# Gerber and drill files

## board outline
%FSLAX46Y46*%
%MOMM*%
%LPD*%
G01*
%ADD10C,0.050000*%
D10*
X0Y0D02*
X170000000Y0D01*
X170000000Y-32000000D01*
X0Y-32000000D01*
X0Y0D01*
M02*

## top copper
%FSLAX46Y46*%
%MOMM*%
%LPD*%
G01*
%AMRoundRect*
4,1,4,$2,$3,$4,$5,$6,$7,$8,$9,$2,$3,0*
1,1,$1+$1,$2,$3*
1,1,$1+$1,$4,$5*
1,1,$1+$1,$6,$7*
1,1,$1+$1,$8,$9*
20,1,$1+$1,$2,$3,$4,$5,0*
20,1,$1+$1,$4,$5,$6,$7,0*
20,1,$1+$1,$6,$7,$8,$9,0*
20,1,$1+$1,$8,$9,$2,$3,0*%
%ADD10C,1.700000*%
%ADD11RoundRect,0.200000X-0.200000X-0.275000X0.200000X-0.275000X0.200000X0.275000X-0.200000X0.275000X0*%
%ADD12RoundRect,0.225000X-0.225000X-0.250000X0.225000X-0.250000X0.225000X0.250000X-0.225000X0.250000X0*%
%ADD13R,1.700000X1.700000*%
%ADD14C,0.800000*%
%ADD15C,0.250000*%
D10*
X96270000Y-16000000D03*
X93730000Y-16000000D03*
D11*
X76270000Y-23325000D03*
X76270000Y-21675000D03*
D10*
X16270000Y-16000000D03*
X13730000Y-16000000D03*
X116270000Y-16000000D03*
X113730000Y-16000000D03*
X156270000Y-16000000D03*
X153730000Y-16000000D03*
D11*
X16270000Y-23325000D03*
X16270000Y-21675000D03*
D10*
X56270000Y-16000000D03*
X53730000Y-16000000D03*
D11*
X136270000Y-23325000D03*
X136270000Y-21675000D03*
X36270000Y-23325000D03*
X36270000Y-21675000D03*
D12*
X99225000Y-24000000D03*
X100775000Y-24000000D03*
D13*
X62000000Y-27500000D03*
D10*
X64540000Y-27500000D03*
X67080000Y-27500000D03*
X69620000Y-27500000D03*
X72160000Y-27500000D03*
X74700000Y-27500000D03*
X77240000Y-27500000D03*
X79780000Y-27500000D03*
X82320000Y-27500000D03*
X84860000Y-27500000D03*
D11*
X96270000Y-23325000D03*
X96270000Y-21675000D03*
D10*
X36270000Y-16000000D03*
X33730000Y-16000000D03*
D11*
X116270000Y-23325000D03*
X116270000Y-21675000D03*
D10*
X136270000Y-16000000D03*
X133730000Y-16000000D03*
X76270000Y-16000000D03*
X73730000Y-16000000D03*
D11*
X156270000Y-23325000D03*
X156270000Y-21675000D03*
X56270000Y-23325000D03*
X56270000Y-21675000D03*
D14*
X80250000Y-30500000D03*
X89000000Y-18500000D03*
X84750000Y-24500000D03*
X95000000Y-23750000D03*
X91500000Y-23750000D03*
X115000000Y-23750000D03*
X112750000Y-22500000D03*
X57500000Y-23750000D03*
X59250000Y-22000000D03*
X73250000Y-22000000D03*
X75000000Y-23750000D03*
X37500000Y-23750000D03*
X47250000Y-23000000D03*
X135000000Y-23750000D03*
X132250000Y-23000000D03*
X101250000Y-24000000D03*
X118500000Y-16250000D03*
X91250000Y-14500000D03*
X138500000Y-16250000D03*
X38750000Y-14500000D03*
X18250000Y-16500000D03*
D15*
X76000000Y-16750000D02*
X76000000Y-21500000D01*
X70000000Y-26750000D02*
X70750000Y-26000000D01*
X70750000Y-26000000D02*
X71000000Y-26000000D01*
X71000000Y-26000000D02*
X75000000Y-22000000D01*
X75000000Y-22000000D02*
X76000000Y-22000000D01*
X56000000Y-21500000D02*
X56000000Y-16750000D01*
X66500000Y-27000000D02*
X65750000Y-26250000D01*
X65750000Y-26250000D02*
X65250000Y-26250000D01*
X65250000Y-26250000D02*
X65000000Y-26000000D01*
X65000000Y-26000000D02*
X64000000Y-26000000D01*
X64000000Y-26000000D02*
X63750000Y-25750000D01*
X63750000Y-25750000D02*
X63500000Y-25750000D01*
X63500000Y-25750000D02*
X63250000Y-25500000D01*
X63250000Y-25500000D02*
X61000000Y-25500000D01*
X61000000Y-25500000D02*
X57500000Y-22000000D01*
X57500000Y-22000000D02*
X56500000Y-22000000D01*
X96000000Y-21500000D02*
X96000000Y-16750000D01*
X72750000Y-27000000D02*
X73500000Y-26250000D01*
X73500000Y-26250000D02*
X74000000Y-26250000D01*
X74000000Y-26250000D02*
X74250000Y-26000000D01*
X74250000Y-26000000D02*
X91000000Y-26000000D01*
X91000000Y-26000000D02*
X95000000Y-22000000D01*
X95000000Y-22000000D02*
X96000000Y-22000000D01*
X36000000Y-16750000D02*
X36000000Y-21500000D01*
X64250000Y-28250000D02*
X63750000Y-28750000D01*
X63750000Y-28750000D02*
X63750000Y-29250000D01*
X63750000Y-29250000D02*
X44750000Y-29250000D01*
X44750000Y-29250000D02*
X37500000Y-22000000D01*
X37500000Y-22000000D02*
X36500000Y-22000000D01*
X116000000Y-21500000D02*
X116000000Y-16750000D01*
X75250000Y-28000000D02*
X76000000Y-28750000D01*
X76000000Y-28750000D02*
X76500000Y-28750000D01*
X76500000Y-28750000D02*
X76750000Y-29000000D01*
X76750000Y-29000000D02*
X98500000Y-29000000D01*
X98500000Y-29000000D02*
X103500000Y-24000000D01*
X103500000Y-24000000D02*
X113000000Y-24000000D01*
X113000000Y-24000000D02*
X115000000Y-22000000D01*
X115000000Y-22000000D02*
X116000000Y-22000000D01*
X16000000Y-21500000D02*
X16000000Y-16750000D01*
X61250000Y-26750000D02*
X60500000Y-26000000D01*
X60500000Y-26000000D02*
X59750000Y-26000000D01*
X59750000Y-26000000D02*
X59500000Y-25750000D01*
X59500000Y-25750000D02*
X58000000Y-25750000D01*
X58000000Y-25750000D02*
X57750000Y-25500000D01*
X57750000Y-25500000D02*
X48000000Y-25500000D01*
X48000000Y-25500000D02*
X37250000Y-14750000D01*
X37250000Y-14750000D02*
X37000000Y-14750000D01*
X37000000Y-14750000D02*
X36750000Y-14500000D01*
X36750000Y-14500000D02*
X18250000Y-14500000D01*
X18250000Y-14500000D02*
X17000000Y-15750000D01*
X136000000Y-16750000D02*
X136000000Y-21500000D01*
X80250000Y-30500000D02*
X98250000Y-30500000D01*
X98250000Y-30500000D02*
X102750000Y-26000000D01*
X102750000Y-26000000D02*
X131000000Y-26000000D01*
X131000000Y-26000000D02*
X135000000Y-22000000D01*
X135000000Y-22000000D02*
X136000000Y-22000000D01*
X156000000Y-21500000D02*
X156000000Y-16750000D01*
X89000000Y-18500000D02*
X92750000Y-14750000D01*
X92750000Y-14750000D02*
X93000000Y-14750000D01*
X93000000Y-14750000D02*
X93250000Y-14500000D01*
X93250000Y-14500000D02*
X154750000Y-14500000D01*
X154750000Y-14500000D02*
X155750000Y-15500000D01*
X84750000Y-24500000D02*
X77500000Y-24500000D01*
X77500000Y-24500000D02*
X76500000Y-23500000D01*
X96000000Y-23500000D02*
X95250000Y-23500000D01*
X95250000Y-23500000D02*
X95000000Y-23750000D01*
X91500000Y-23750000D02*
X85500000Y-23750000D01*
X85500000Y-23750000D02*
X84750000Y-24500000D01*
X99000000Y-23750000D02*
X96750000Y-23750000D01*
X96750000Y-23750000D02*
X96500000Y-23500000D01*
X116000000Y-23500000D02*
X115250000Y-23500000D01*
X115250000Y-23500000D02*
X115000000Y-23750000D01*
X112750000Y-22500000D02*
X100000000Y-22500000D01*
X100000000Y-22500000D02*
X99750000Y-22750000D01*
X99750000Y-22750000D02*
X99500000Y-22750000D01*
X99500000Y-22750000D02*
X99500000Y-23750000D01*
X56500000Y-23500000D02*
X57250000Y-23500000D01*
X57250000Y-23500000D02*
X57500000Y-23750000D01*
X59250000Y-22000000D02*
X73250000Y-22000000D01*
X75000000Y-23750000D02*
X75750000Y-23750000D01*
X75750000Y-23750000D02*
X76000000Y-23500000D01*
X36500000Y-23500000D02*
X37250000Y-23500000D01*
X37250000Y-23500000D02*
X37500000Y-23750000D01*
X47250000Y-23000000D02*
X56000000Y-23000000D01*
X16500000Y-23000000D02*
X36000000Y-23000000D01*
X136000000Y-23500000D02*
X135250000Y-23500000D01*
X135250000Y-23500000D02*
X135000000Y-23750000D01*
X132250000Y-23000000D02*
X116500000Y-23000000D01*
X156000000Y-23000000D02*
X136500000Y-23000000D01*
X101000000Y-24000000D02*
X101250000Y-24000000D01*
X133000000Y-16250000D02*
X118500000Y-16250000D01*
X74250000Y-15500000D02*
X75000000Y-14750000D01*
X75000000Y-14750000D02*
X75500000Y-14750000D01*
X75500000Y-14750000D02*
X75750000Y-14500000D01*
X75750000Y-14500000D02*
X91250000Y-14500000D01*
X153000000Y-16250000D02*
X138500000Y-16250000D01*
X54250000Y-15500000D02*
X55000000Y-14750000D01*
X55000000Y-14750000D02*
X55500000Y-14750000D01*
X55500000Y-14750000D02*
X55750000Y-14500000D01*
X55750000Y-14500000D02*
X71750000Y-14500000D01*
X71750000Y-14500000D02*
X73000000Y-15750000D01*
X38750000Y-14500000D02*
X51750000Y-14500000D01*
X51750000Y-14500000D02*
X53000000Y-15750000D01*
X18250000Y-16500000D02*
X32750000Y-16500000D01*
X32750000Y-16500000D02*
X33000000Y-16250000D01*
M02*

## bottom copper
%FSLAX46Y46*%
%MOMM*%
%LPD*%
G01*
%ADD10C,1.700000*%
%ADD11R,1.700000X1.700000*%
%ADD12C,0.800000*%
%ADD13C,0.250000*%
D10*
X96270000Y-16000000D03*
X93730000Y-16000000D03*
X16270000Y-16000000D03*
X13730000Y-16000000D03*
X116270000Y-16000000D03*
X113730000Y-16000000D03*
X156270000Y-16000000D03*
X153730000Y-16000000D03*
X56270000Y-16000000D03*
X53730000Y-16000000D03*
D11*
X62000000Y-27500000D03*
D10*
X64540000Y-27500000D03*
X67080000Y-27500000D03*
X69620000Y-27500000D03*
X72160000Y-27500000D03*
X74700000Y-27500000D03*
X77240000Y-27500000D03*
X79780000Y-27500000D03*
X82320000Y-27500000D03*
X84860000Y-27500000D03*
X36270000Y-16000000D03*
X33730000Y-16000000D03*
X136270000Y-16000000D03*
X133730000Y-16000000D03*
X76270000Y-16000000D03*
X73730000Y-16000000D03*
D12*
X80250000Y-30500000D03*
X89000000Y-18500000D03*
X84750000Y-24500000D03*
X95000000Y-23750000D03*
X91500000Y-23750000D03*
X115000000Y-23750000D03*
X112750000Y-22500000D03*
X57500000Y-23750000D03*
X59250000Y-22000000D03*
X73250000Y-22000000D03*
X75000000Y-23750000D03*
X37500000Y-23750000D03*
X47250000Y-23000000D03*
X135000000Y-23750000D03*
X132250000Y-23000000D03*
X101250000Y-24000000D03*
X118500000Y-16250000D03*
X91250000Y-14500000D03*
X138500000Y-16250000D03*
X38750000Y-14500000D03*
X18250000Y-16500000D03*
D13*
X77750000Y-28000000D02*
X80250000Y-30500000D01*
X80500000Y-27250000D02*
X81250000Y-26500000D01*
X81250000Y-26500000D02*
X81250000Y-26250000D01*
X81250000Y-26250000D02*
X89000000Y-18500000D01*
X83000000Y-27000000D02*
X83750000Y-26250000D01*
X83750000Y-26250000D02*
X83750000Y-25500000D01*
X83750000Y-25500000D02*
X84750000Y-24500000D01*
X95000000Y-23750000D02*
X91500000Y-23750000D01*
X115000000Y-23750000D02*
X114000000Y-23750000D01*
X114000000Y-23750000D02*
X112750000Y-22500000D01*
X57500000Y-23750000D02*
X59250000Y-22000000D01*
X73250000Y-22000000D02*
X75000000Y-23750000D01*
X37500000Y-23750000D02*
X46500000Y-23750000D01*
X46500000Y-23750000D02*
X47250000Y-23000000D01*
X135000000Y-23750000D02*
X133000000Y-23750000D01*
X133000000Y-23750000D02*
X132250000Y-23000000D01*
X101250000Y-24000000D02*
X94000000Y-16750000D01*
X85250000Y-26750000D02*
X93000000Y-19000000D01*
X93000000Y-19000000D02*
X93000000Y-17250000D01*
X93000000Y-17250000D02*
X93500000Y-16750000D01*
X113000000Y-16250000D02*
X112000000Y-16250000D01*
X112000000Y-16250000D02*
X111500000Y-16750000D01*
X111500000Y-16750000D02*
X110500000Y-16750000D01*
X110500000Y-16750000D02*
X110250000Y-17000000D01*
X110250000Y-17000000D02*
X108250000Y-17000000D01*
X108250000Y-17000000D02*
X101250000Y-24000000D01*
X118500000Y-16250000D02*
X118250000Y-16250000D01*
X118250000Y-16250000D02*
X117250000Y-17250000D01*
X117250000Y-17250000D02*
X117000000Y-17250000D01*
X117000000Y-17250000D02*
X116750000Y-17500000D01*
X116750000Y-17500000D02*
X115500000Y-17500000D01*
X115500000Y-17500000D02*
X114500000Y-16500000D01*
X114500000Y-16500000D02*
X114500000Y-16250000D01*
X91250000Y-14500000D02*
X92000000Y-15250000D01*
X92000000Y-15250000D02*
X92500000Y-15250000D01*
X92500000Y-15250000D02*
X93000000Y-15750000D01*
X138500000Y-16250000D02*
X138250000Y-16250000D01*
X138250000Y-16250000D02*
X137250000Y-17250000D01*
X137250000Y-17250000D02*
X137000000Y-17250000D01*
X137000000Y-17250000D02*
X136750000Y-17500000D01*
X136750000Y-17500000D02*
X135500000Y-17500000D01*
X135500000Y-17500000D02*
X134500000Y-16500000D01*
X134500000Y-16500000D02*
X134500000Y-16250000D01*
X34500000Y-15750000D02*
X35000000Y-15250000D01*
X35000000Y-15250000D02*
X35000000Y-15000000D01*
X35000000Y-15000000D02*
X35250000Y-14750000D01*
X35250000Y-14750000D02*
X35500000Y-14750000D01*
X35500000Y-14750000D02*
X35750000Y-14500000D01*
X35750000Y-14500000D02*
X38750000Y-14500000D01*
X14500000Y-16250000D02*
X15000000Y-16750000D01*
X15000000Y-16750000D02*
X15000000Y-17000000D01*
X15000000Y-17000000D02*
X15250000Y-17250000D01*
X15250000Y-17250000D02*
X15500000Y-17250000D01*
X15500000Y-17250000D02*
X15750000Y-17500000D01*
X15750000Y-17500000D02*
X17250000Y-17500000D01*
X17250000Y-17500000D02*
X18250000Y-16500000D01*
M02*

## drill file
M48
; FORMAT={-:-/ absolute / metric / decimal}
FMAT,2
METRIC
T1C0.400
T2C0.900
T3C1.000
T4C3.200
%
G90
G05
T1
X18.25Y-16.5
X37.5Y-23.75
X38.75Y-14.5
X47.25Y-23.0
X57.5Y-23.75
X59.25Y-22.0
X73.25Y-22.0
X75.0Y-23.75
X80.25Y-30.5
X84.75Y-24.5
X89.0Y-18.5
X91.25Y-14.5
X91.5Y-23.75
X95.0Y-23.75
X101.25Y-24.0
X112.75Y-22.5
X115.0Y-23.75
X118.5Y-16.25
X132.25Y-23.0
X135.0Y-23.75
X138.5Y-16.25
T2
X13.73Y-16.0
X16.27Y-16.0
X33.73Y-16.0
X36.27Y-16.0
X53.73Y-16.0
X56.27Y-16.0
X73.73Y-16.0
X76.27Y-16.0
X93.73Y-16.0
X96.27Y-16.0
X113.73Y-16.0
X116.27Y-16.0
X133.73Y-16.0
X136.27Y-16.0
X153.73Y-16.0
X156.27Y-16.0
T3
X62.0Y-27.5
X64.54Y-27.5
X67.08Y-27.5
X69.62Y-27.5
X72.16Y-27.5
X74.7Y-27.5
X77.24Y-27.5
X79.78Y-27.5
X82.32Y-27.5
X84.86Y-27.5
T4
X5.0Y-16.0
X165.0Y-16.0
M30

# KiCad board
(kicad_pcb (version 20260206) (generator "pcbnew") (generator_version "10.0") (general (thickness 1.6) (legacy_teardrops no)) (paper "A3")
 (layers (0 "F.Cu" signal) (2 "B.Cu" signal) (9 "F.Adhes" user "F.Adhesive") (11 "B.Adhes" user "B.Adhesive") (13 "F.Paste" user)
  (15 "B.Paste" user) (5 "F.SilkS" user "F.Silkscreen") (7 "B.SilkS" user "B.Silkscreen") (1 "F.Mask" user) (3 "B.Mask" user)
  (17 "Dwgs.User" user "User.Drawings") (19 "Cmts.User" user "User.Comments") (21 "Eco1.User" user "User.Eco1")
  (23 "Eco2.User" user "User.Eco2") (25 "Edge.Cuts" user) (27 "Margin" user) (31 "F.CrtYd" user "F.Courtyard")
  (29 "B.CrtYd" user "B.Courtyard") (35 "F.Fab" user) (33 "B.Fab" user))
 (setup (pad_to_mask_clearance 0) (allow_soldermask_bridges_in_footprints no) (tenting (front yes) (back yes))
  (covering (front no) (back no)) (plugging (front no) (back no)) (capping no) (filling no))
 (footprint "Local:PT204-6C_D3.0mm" (layer "F.Cu") (at 95 16)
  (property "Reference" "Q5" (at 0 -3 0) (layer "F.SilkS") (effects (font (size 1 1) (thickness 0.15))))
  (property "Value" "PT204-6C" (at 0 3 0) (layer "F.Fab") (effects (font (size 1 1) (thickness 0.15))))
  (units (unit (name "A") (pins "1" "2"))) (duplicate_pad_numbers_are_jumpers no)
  (pad "1" thru_hole circle (at 1.27 0) (size 1.7 1.7) (drill 0.9) (layers "*.Cu" "*.Mask") (remove_unused_layers no) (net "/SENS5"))
  (pad "2" thru_hole circle (at -1.27 0) (size 1.7 1.7) (drill 0.9) (layers "*.Cu" "*.Mask") (remove_unused_layers no) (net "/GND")))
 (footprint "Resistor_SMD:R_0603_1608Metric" (layer "F.Cu") (at 76.27 22.5 90)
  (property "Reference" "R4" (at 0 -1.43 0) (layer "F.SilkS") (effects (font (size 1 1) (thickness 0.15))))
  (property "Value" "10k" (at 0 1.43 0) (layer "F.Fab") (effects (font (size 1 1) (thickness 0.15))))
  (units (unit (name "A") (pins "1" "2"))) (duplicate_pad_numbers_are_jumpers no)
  (pad "1" smd roundrect (at -0.825 0) (size 0.8 0.95) (layers "F.Cu" "F.Mask" "F.Paste") (roundrect_rratio 0.25) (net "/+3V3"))
  (pad "2" smd roundrect (at 0.825 0) (size 0.8 0.95) (layers "F.Cu" "F.Mask" "F.Paste") (roundrect_rratio 0.25) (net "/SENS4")))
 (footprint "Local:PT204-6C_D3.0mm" (layer "F.Cu") (at 15 16)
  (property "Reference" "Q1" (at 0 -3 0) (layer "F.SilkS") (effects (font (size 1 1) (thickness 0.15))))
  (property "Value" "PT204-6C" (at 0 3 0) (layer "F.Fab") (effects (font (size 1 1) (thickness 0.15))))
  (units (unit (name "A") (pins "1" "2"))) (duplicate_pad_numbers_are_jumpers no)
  (pad "1" thru_hole circle (at 1.27 0) (size 1.7 1.7) (drill 0.9) (layers "*.Cu" "*.Mask") (remove_unused_layers no) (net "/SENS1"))
  (pad "2" thru_hole circle (at -1.27 0) (size 1.7 1.7) (drill 0.9) (layers "*.Cu" "*.Mask") (remove_unused_layers no) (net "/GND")))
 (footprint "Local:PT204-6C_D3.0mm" (layer "F.Cu") (at 115 16)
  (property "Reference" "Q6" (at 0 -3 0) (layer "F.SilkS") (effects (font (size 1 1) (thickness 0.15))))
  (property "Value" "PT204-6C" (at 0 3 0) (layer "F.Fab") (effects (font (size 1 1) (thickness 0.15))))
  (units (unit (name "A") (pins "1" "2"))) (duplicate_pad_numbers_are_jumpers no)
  (pad "1" thru_hole circle (at 1.27 0) (size 1.7 1.7) (drill 0.9) (layers "*.Cu" "*.Mask") (remove_unused_layers no) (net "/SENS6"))
  (pad "2" thru_hole circle (at -1.27 0) (size 1.7 1.7) (drill 0.9) (layers "*.Cu" "*.Mask") (remove_unused_layers no) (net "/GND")))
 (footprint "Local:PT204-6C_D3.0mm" (layer "F.Cu") (at 155 16)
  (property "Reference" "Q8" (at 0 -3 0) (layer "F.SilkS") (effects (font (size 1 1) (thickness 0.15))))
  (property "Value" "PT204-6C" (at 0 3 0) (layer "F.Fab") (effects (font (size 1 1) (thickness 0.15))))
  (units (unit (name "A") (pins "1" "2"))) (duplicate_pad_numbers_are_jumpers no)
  (pad "1" thru_hole circle (at 1.27 0) (size 1.7 1.7) (drill 0.9) (layers "*.Cu" "*.Mask") (remove_unused_layers no) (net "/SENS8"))
  (pad "2" thru_hole circle (at -1.27 0) (size 1.7 1.7) (drill 0.9) (layers "*.Cu" "*.Mask") (remove_unused_layers no) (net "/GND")))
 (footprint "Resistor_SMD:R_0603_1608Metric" (layer "F.Cu") (at 16.27 22.5 90)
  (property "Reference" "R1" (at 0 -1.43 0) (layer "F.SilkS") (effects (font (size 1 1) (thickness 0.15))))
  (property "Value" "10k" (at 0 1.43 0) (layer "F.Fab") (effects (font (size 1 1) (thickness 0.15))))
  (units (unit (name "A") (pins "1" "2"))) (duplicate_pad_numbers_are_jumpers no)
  (pad "1" smd roundrect (at -0.825 0) (size 0.8 0.95) (layers "F.Cu" "F.Mask" "F.Paste") (roundrect_rratio 0.25) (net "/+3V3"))
  (pad "2" smd roundrect (at 0.825 0) (size 0.8 0.95) (layers "F.Cu" "F.Mask" "F.Paste") (roundrect_rratio 0.25) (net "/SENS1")))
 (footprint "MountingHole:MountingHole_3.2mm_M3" (layer "F.Cu") (at 5 16)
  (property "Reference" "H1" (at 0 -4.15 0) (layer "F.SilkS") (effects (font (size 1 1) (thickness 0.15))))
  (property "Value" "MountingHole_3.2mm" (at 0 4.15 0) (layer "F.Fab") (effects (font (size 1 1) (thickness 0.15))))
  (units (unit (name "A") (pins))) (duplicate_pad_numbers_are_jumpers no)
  (pad "" np_thru_hole circle (at 0 0) (size 3.2 3.2) (drill 3.2) (layers "*.Cu" "*.Mask")))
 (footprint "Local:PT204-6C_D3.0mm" (layer "F.Cu") (at 55 16)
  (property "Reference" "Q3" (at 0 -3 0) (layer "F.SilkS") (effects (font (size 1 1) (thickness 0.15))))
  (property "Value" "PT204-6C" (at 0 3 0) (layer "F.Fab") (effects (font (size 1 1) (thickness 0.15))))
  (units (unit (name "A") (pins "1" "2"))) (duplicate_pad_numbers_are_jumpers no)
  (pad "1" thru_hole circle (at 1.27 0) (size 1.7 1.7) (drill 0.9) (layers "*.Cu" "*.Mask") (remove_unused_layers no) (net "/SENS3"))
  (pad "2" thru_hole circle (at -1.27 0) (size 1.7 1.7) (drill 0.9) (layers "*.Cu" "*.Mask") (remove_unused_layers no) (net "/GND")))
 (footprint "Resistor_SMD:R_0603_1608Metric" (layer "F.Cu") (at 136.27 22.5 90)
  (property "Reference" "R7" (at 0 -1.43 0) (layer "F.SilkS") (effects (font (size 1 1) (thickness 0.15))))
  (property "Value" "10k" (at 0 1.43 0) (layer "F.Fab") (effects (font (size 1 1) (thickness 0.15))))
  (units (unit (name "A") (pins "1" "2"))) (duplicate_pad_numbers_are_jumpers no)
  (pad "1" smd roundrect (at -0.825 0) (size 0.8 0.95) (layers "F.Cu" "F.Mask" "F.Paste") (roundrect_rratio 0.25) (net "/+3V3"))
  (pad "2" smd roundrect (at 0.825 0) (size 0.8 0.95) (layers "F.Cu" "F.Mask" "F.Paste") (roundrect_rratio 0.25) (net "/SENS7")))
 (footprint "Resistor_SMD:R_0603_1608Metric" (layer "F.Cu") (at 36.27 22.5 90)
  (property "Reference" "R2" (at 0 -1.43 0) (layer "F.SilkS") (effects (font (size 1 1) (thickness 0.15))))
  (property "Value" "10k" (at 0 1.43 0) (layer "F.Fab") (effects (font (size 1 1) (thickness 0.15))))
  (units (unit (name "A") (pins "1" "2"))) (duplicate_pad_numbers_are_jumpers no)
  (pad "1" smd roundrect (at -0.825 0) (size 0.8 0.95) (layers "F.Cu" "F.Mask" "F.Paste") (roundrect_rratio 0.25) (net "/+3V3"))
  (pad "2" smd roundrect (at 0.825 0) (size 0.8 0.95) (layers "F.Cu" "F.Mask" "F.Paste") (roundrect_rratio 0.25) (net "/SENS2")))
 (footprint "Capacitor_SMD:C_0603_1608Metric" (layer "F.Cu") (at 100 24)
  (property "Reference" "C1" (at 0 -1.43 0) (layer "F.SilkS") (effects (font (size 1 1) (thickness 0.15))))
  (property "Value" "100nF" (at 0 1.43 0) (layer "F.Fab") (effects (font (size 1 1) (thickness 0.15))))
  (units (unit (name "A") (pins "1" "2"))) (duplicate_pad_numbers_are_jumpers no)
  (pad "1" smd roundrect (at -0.775 0) (size 0.9 0.95) (layers "F.Cu" "F.Mask" "F.Paste") (roundrect_rratio 0.25) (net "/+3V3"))
  (pad "2" smd roundrect (at 0.775 0) (size 0.9 0.95) (layers "F.Cu" "F.Mask" "F.Paste") (roundrect_rratio 0.25) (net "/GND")))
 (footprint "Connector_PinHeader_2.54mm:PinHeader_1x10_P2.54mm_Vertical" (layer "F.Cu") (at 62 27.5 90)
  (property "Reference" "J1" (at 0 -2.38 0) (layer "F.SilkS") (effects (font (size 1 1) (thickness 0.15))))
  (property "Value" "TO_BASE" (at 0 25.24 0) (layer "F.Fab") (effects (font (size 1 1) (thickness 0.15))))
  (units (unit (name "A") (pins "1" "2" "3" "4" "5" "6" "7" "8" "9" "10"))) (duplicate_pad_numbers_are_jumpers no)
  (pad "1" thru_hole rect (at 0 0) (size 1.7 1.7) (drill 1) (layers "*.Cu" "*.Mask") (remove_unused_layers no) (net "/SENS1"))
  (pad "2" thru_hole circle (at 0 2.54) (size 1.7 1.7) (drill 1) (layers "*.Cu" "*.Mask") (remove_unused_layers no) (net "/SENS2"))
  (pad "3" thru_hole circle (at 0 5.08) (size 1.7 1.7) (drill 1) (layers "*.Cu" "*.Mask") (remove_unused_layers no) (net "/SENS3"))
  (pad "4" thru_hole circle (at 0 7.62) (size 1.7 1.7) (drill 1) (layers "*.Cu" "*.Mask") (remove_unused_layers no) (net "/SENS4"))
  (pad "5" thru_hole circle (at 0 10.16) (size 1.7 1.7) (drill 1) (layers "*.Cu" "*.Mask") (remove_unused_layers no) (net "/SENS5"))
  (pad "6" thru_hole circle (at 0 12.7) (size 1.7 1.7) (drill 1) (layers "*.Cu" "*.Mask") (remove_unused_layers no) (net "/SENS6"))
  (pad "7" thru_hole circle (at 0 15.24) (size 1.7 1.7) (drill 1) (layers "*.Cu" "*.Mask") (remove_unused_layers no) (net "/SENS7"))
  (pad "8" thru_hole circle (at 0 17.78) (size 1.7 1.7) (drill 1) (layers "*.Cu" "*.Mask") (remove_unused_layers no) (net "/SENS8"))
  (pad "9" thru_hole circle (at 0 20.32) (size 1.7 1.7) (drill 1) (layers "*.Cu" "*.Mask") (remove_unused_layers no) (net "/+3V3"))
  (pad "10" thru_hole circle (at 0 22.86) (size 1.7 1.7) (drill 1) (layers "*.Cu" "*.Mask") (remove_unused_layers no) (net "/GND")))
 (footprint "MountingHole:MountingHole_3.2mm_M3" (layer "F.Cu") (at 165 16)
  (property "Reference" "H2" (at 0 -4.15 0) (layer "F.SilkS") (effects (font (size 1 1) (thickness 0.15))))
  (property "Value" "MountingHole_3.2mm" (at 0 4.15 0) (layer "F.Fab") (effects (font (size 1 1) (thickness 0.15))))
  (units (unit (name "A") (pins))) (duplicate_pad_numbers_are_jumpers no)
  (pad "" np_thru_hole circle (at 0 0) (size 3.2 3.2) (drill 3.2) (layers "*.Cu" "*.Mask")))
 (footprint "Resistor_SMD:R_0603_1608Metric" (layer "F.Cu") (at 96.27 22.5 90)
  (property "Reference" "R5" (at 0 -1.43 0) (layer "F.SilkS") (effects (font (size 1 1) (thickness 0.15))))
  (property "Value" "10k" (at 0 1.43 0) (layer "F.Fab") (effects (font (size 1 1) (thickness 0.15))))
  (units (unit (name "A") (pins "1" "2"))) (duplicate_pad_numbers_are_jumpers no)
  (pad "1" smd roundrect (at -0.825 0) (size 0.8 0.95) (layers "F.Cu" "F.Mask" "F.Paste") (roundrect_rratio 0.25) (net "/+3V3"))
  (pad "2" smd roundrect (at 0.825 0) (size 0.8 0.95) (layers "F.Cu" "F.Mask" "F.Paste") (roundrect_rratio 0.25) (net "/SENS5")))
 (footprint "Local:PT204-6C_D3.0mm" (layer "F.Cu") (at 35 16)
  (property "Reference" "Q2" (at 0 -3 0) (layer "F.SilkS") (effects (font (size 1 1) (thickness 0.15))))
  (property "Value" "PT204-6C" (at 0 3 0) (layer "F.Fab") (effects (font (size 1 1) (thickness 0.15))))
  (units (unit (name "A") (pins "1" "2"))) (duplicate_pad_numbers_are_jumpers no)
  (pad "1" thru_hole circle (at 1.27 0) (size 1.7 1.7) (drill 0.9) (layers "*.Cu" "*.Mask") (remove_unused_layers no) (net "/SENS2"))
  (pad "2" thru_hole circle (at -1.27 0) (size 1.7 1.7) (drill 0.9) (layers "*.Cu" "*.Mask") (remove_unused_layers no) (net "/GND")))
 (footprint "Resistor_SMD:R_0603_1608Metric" (layer "F.Cu") (at 116.27 22.5 90)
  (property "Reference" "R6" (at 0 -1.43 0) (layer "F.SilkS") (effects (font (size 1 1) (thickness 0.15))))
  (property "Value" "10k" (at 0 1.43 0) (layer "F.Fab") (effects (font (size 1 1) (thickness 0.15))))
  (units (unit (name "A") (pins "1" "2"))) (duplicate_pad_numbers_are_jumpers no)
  (pad "1" smd roundrect (at -0.825 0) (size 0.8 0.95) (layers "F.Cu" "F.Mask" "F.Paste") (roundrect_rratio 0.25) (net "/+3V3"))
  (pad "2" smd roundrect (at 0.825 0) (size 0.8 0.95) (layers "F.Cu" "F.Mask" "F.Paste") (roundrect_rratio 0.25) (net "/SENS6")))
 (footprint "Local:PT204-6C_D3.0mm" (layer "F.Cu") (at 135 16)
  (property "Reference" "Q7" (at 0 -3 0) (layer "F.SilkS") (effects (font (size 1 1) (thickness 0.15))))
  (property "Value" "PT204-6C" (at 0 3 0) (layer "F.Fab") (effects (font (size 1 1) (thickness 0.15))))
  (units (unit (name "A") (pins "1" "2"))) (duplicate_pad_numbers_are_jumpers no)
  (pad "1" thru_hole circle (at 1.27 0) (size 1.7 1.7) (drill 0.9) (layers "*.Cu" "*.Mask") (remove_unused_layers no) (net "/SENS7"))
  (pad "2" thru_hole circle (at -1.27 0) (size 1.7 1.7) (drill 0.9) (layers "*.Cu" "*.Mask") (remove_unused_layers no) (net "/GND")))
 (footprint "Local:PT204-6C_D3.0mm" (layer "F.Cu") (at 75 16)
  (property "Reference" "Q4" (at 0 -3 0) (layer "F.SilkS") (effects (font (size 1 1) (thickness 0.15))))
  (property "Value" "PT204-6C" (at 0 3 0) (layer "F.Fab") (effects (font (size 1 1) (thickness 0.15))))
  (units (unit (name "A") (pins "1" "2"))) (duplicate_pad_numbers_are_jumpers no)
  (pad "1" thru_hole circle (at 1.27 0) (size 1.7 1.7) (drill 0.9) (layers "*.Cu" "*.Mask") (remove_unused_layers no) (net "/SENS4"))
  (pad "2" thru_hole circle (at -1.27 0) (size 1.7 1.7) (drill 0.9) (layers "*.Cu" "*.Mask") (remove_unused_layers no) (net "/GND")))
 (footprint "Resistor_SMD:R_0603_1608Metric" (layer "F.Cu") (at 156.27 22.5 90)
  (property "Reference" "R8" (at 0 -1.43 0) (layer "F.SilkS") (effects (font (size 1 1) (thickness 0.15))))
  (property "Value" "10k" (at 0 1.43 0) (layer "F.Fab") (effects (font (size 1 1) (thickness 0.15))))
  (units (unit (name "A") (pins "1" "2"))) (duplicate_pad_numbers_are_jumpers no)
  (pad "1" smd roundrect (at -0.825 0) (size 0.8 0.95) (layers "F.Cu" "F.Mask" "F.Paste") (roundrect_rratio 0.25) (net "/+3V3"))
  (pad "2" smd roundrect (at 0.825 0) (size 0.8 0.95) (layers "F.Cu" "F.Mask" "F.Paste") (roundrect_rratio 0.25) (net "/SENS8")))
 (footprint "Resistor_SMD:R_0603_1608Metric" (layer "F.Cu") (at 56.27 22.5 90)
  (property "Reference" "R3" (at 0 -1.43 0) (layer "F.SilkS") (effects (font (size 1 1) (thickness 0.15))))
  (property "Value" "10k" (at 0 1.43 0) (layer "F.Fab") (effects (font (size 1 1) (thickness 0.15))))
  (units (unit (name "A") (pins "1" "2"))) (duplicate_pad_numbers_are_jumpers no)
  (pad "1" smd roundrect (at -0.825 0) (size 0.8 0.95) (layers "F.Cu" "F.Mask" "F.Paste") (roundrect_rratio 0.25) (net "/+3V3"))
  (pad "2" smd roundrect (at 0.825 0) (size 0.8 0.95) (layers "F.Cu" "F.Mask" "F.Paste") (roundrect_rratio 0.25) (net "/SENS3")))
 (gr_rect (start 0 0) (end 170 32) (stroke (width 0.05) (type solid)) (fill no) (layer "Edge.Cuts"))
 (segment (start 76 16.75) (end 76 21.5) (width 0.25) (layer "F.Cu") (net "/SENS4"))
 (segment (start 70 26.75) (end 70.75 26) (width 0.25) (layer "F.Cu") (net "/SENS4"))
 (segment (start 70.75 26) (end 71 26) (width 0.25) (layer "F.Cu") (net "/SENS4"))
 (segment (start 71 26) (end 75 22) (width 0.25) (layer "F.Cu") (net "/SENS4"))
 (segment (start 75 22) (end 76 22) (width 0.25) (layer "F.Cu") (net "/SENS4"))
 (segment (start 56 21.5) (end 56 16.75) (width 0.25) (layer "F.Cu") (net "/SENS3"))
 (segment (start 66.5 27) (end 65.75 26.25) (width 0.25) (layer "F.Cu") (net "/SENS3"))
 (segment (start 65.75 26.25) (end 65.25 26.25) (width 0.25) (layer "F.Cu") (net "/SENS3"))
 (segment (start 65.25 26.25) (end 65 26) (width 0.25) (layer "F.Cu") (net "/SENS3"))
 (segment (start 65 26) (end 64 26) (width 0.25) (layer "F.Cu") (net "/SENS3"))
 (segment (start 64 26) (end 63.75 25.75) (width 0.25) (layer "F.Cu") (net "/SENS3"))
 (segment (start 63.75 25.75) (end 63.5 25.75) (width 0.25) (layer "F.Cu") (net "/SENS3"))
 (segment (start 63.5 25.75) (end 63.25 25.5) (width 0.25) (layer "F.Cu") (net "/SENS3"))
 (segment (start 63.25 25.5) (end 61 25.5) (width 0.25) (layer "F.Cu") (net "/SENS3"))
 (segment (start 61 25.5) (end 57.5 22) (width 0.25) (layer "F.Cu") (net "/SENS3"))
 (segment (start 57.5 22) (end 56.5 22) (width 0.25) (layer "F.Cu") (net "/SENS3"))
 (segment (start 96 21.5) (end 96 16.75) (width 0.25) (layer "F.Cu") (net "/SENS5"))
 (segment (start 72.75 27) (end 73.5 26.25) (width 0.25) (layer "F.Cu") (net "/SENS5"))
 (segment (start 73.5 26.25) (end 74 26.25) (width 0.25) (layer "F.Cu") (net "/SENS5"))
 (segment (start 74 26.25) (end 74.25 26) (width 0.25) (layer "F.Cu") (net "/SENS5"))
 (segment (start 74.25 26) (end 91 26) (width 0.25) (layer "F.Cu") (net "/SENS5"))
 (segment (start 91 26) (end 95 22) (width 0.25) (layer "F.Cu") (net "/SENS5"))
 (segment (start 95 22) (end 96 22) (width 0.25) (layer "F.Cu") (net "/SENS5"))
 (segment (start 36 16.75) (end 36 21.5) (width 0.25) (layer "F.Cu") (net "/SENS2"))
 (segment (start 64.25 28.25) (end 63.75 28.75) (width 0.25) (layer "F.Cu") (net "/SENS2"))
 (segment (start 63.75 28.75) (end 63.75 29.25) (width 0.25) (layer "F.Cu") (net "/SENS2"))
 (segment (start 63.75 29.25) (end 44.75 29.25) (width 0.25) (layer "F.Cu") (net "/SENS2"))
 (segment (start 44.75 29.25) (end 37.5 22) (width 0.25) (layer "F.Cu") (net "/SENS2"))
 (segment (start 37.5 22) (end 36.5 22) (width 0.25) (layer "F.Cu") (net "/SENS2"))
 (segment (start 116 21.5) (end 116 16.75) (width 0.25) (layer "F.Cu") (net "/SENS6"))
 (segment (start 75.25 28) (end 76 28.75) (width 0.25) (layer "F.Cu") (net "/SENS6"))
 (segment (start 76 28.75) (end 76.5 28.75) (width 0.25) (layer "F.Cu") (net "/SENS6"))
 (segment (start 76.5 28.75) (end 76.75 29) (width 0.25) (layer "F.Cu") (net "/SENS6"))
 (segment (start 76.75 29) (end 98.5 29) (width 0.25) (layer "F.Cu") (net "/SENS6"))
 (segment (start 98.5 29) (end 103.5 24) (width 0.25) (layer "F.Cu") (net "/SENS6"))
 (segment (start 103.5 24) (end 113 24) (width 0.25) (layer "F.Cu") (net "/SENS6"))
 (segment (start 113 24) (end 115 22) (width 0.25) (layer "F.Cu") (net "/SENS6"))
 (segment (start 115 22) (end 116 22) (width 0.25) (layer "F.Cu") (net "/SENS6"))
 (segment (start 16 21.5) (end 16 16.75) (width 0.25) (layer "F.Cu") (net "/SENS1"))
 (segment (start 61.25 26.75) (end 60.5 26) (width 0.25) (layer "F.Cu") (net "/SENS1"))
 (segment (start 60.5 26) (end 59.75 26) (width 0.25) (layer "F.Cu") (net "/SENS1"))
 (segment (start 59.75 26) (end 59.5 25.75) (width 0.25) (layer "F.Cu") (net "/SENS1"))
 (segment (start 59.5 25.75) (end 58 25.75) (width 0.25) (layer "F.Cu") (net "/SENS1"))
 (segment (start 58 25.75) (end 57.75 25.5) (width 0.25) (layer "F.Cu") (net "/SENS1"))
 (segment (start 57.75 25.5) (end 48 25.5) (width 0.25) (layer "F.Cu") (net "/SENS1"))
 (segment (start 48 25.5) (end 37.25 14.75) (width 0.25) (layer "F.Cu") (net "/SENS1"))
 (segment (start 37.25 14.75) (end 37 14.75) (width 0.25) (layer "F.Cu") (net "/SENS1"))
 (segment (start 37 14.75) (end 36.75 14.5) (width 0.25) (layer "F.Cu") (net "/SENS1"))
 (segment (start 36.75 14.5) (end 18.25 14.5) (width 0.25) (layer "F.Cu") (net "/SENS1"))
 (segment (start 18.25 14.5) (end 17 15.75) (width 0.25) (layer "F.Cu") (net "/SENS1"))
 (segment (start 136 16.75) (end 136 21.5) (width 0.25) (layer "F.Cu") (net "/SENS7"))
 (segment (start 77.75 28) (end 80.25 30.5) (width 0.25) (layer "B.Cu") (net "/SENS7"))
 (segment (start 80.25 30.5) (end 98.25 30.5) (width 0.25) (layer "F.Cu") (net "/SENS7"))
 (segment (start 98.25 30.5) (end 102.75 26) (width 0.25) (layer "F.Cu") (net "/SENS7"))
 (segment (start 102.75 26) (end 131 26) (width 0.25) (layer "F.Cu") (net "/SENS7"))
 (segment (start 131 26) (end 135 22) (width 0.25) (layer "F.Cu") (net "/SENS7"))
 (segment (start 135 22) (end 136 22) (width 0.25) (layer "F.Cu") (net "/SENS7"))
 (segment (start 156 21.5) (end 156 16.75) (width 0.25) (layer "F.Cu") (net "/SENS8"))
 (segment (start 80.5 27.25) (end 81.25 26.5) (width 0.25) (layer "B.Cu") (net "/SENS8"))
 (segment (start 81.25 26.5) (end 81.25 26.25) (width 0.25) (layer "B.Cu") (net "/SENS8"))
 (segment (start 81.25 26.25) (end 89 18.5) (width 0.25) (layer "B.Cu") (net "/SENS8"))
 (segment (start 89 18.5) (end 92.75 14.75) (width 0.25) (layer "F.Cu") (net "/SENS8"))
 (segment (start 92.75 14.75) (end 93 14.75) (width 0.25) (layer "F.Cu") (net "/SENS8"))
 (segment (start 93 14.75) (end 93.25 14.5) (width 0.25) (layer "F.Cu") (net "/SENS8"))
 (segment (start 93.25 14.5) (end 154.75 14.5) (width 0.25) (layer "F.Cu") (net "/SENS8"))
 (segment (start 154.75 14.5) (end 155.75 15.5) (width 0.25) (layer "F.Cu") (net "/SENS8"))
 (segment (start 83 27) (end 83.75 26.25) (width 0.25) (layer "B.Cu") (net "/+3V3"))
 (segment (start 83.75 26.25) (end 83.75 25.5) (width 0.25) (layer "B.Cu") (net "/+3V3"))
 (segment (start 83.75 25.5) (end 84.75 24.5) (width 0.25) (layer "B.Cu") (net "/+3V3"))
 (segment (start 84.75 24.5) (end 77.5 24.5) (width 0.25) (layer "F.Cu") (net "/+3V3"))
 (segment (start 77.5 24.5) (end 76.5 23.5) (width 0.25) (layer "F.Cu") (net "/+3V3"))
 (segment (start 96 23.5) (end 95.25 23.5) (width 0.25) (layer "F.Cu") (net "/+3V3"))
 (segment (start 95.25 23.5) (end 95 23.75) (width 0.25) (layer "F.Cu") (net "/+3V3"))
 (segment (start 95 23.75) (end 91.5 23.75) (width 0.25) (layer "B.Cu") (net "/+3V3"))
 (segment (start 91.5 23.75) (end 85.5 23.75) (width 0.25) (layer "F.Cu") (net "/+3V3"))
 (segment (start 85.5 23.75) (end 84.75 24.5) (width 0.25) (layer "F.Cu") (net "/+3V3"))
 (segment (start 99 23.75) (end 96.75 23.75) (width 0.25) (layer "F.Cu") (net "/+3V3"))
 (segment (start 96.75 23.75) (end 96.5 23.5) (width 0.25) (layer "F.Cu") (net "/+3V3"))
 (segment (start 116 23.5) (end 115.25 23.5) (width 0.25) (layer "F.Cu") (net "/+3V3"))
 (segment (start 115.25 23.5) (end 115 23.75) (width 0.25) (layer "F.Cu") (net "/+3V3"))
 (segment (start 115 23.75) (end 114 23.75) (width 0.25) (layer "B.Cu") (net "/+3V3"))
 (segment (start 114 23.75) (end 112.75 22.5) (width 0.25) (layer "B.Cu") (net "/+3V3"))
 (segment (start 112.75 22.5) (end 100 22.5) (width 0.25) (layer "F.Cu") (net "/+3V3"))
 (segment (start 100 22.5) (end 99.75 22.75) (width 0.25) (layer "F.Cu") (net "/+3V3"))
 (segment (start 99.75 22.75) (end 99.5 22.75) (width 0.25) (layer "F.Cu") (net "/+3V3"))
 (segment (start 99.5 22.75) (end 99.5 23.75) (width 0.25) (layer "F.Cu") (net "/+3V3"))
 (segment (start 56.5 23.5) (end 57.25 23.5) (width 0.25) (layer "F.Cu") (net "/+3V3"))
 (segment (start 57.25 23.5) (end 57.5 23.75) (width 0.25) (layer "F.Cu") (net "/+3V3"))
 (segment (start 57.5 23.75) (end 59.25 22) (width 0.25) (layer "B.Cu") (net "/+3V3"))
 (segment (start 59.25 22) (end 73.25 22) (width 0.25) (layer "F.Cu") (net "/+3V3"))
 (segment (start 73.25 22) (end 75 23.75) (width 0.25) (layer "B.Cu") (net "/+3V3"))
 (segment (start 75 23.75) (end 75.75 23.75) (width 0.25) (layer "F.Cu") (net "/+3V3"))
 (segment (start 75.75 23.75) (end 76 23.5) (width 0.25) (layer "F.Cu") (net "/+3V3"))
 (segment (start 36.5 23.5) (end 37.25 23.5) (width 0.25) (layer "F.Cu") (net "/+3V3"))
 (segment (start 37.25 23.5) (end 37.5 23.75) (width 0.25) (layer "F.Cu") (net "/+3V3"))
 (segment (start 37.5 23.75) (end 46.5 23.75) (width 0.25) (layer "B.Cu") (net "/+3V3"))
 (segment (start 46.5 23.75) (end 47.25 23) (width 0.25) (layer "B.Cu") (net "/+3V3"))
 (segment (start 47.25 23) (end 56 23) (width 0.25) (layer "F.Cu") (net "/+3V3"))
 (segment (start 16.5 23) (end 36 23) (width 0.25) (layer "F.Cu") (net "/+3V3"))
 (segment (start 136 23.5) (end 135.25 23.5) (width 0.25) (layer "F.Cu") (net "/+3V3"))
 (segment (start 135.25 23.5) (end 135 23.75) (width 0.25) (layer "F.Cu") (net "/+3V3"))
 (segment (start 135 23.75) (end 133 23.75) (width 0.25) (layer "B.Cu") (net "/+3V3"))
 (segment (start 133 23.75) (end 132.25 23) (width 0.25) (layer "B.Cu") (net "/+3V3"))
 (segment (start 132.25 23) (end 116.5 23) (width 0.25) (layer "F.Cu") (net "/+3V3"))
 (segment (start 156 23) (end 136.5 23) (width 0.25) (layer "F.Cu") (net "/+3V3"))
 (segment (start 101 24) (end 101.25 24) (width 0.25) (layer "F.Cu") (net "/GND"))
 (segment (start 101.25 24) (end 94 16.75) (width 0.25) (layer "B.Cu") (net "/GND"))
 (segment (start 85.25 26.75) (end 93 19) (width 0.25) (layer "B.Cu") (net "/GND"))
 (segment (start 93 19) (end 93 17.25) (width 0.25) (layer "B.Cu") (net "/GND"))
 (segment (start 93 17.25) (end 93.5 16.75) (width 0.25) (layer "B.Cu") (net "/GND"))
 (segment (start 113 16.25) (end 112 16.25) (width 0.25) (layer "B.Cu") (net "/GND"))
 (segment (start 112 16.25) (end 111.5 16.75) (width 0.25) (layer "B.Cu") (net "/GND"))
 (segment (start 111.5 16.75) (end 110.5 16.75) (width 0.25) (layer "B.Cu") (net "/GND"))
 (segment (start 110.5 16.75) (end 110.25 17) (width 0.25) (layer "B.Cu") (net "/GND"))
 (segment (start 110.25 17) (end 108.25 17) (width 0.25) (layer "B.Cu") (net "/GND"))
 (segment (start 108.25 17) (end 101.25 24) (width 0.25) (layer "B.Cu") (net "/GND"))
 (segment (start 133 16.25) (end 118.5 16.25) (width 0.25) (layer "F.Cu") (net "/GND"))
 (segment (start 118.5 16.25) (end 118.25 16.25) (width 0.25) (layer "B.Cu") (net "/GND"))
 (segment (start 118.25 16.25) (end 117.25 17.25) (width 0.25) (layer "B.Cu") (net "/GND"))
 (segment (start 117.25 17.25) (end 117 17.25) (width 0.25) (layer "B.Cu") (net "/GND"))
 (segment (start 117 17.25) (end 116.75 17.5) (width 0.25) (layer "B.Cu") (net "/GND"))
 (segment (start 116.75 17.5) (end 115.5 17.5) (width 0.25) (layer "B.Cu") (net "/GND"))
 (segment (start 115.5 17.5) (end 114.5 16.5) (width 0.25) (layer "B.Cu") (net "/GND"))
 (segment (start 114.5 16.5) (end 114.5 16.25) (width 0.25) (layer "B.Cu") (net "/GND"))
 (segment (start 74.25 15.5) (end 75 14.75) (width 0.25) (layer "F.Cu") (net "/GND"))
 (segment (start 75 14.75) (end 75.5 14.75) (width 0.25) (layer "F.Cu") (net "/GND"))
 (segment (start 75.5 14.75) (end 75.75 14.5) (width 0.25) (layer "F.Cu") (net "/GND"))
 (segment (start 75.75 14.5) (end 91.25 14.5) (width 0.25) (layer "F.Cu") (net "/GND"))
 (segment (start 91.25 14.5) (end 92 15.25) (width 0.25) (layer "B.Cu") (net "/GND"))
 (segment (start 92 15.25) (end 92.5 15.25) (width 0.25) (layer "B.Cu") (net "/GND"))
 (segment (start 92.5 15.25) (end 93 15.75) (width 0.25) (layer "B.Cu") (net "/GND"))
 (segment (start 153 16.25) (end 138.5 16.25) (width 0.25) (layer "F.Cu") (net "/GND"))
 (segment (start 138.5 16.25) (end 138.25 16.25) (width 0.25) (layer "B.Cu") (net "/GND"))
 (segment (start 138.25 16.25) (end 137.25 17.25) (width 0.25) (layer "B.Cu") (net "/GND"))
 (segment (start 137.25 17.25) (end 137 17.25) (width 0.25) (layer "B.Cu") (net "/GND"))
 (segment (start 137 17.25) (end 136.75 17.5) (width 0.25) (layer "B.Cu") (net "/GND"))
 (segment (start 136.75 17.5) (end 135.5 17.5) (width 0.25) (layer "B.Cu") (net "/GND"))
 (segment (start 135.5 17.5) (end 134.5 16.5) (width 0.25) (layer "B.Cu") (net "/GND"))
 (segment (start 134.5 16.5) (end 134.5 16.25) (width 0.25) (layer "B.Cu") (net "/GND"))
 (segment (start 54.25 15.5) (end 55 14.75) (width 0.25) (layer "F.Cu") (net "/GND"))
 (segment (start 55 14.75) (end 55.5 14.75) (width 0.25) (layer "F.Cu") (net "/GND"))
 (segment (start 55.5 14.75) (end 55.75 14.5) (width 0.25) (layer "F.Cu") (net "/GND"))
 (segment (start 55.75 14.5) (end 71.75 14.5) (width 0.25) (layer "F.Cu") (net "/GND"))
 (segment (start 71.75 14.5) (end 73 15.75) (width 0.25) (layer "F.Cu") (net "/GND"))
 (segment (start 34.5 15.75) (end 35 15.25) (width 0.25) (layer "B.Cu") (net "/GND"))
 (segment (start 35 15.25) (end 35 15) (width 0.25) (layer "B.Cu") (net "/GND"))
 (segment (start 35 15) (end 35.25 14.75) (width 0.25) (layer "B.Cu") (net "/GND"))
 (segment (start 35.25 14.75) (end 35.5 14.75) (width 0.25) (layer "B.Cu") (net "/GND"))
 (segment (start 35.5 14.75) (end 35.75 14.5) (width 0.25) (layer "B.Cu") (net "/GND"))
 (segment (start 35.75 14.5) (end 38.75 14.5) (width 0.25) (layer "B.Cu") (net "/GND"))
 (segment (start 38.75 14.5) (end 51.75 14.5) (width 0.25) (layer "F.Cu") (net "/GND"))
 (segment (start 51.75 14.5) (end 53 15.75) (width 0.25) (layer "F.Cu") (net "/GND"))
 (segment (start 14.5 16.25) (end 15 16.75) (width 0.25) (layer "B.Cu") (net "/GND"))
 (segment (start 15 16.75) (end 15 17) (width 0.25) (layer "B.Cu") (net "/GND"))
 (segment (start 15 17) (end 15.25 17.25) (width 0.25) (layer "B.Cu") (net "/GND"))
 (segment (start 15.25 17.25) (end 15.5 17.25) (width 0.25) (layer "B.Cu") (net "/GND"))
 (segment (start 15.5 17.25) (end 15.75 17.5) (width 0.25) (layer "B.Cu") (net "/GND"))
 (segment (start 15.75 17.5) (end 17.25 17.5) (width 0.25) (layer "B.Cu") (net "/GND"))
 (segment (start 17.25 17.5) (end 18.25 16.5) (width 0.25) (layer "B.Cu") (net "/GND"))
 (segment (start 18.25 16.5) (end 32.75 16.5) (width 0.25) (layer "F.Cu") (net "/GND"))
 (segment (start 32.75 16.5) (end 33 16.25) (width 0.25) (layer "F.Cu") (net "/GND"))
 (via (at 80.25 30.5) (size 0.8) (drill 0.4) (layers "F.Cu" "B.Cu") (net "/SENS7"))
 (via (at 89 18.5) (size 0.8) (drill 0.4) (layers "F.Cu" "B.Cu") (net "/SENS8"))
 (via (at 84.75 24.5) (size 0.8) (drill 0.4) (layers "F.Cu" "B.Cu") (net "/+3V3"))
 (via (at 95 23.75) (size 0.8) (drill 0.4) (layers "F.Cu" "B.Cu") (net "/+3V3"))
 (via (at 91.5 23.75) (size 0.8) (drill 0.4) (layers "F.Cu" "B.Cu") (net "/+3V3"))
 (via (at 115 23.75) (size 0.8) (drill 0.4) (layers "F.Cu" "B.Cu") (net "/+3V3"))
 (via (at 112.75 22.5) (size 0.8) (drill 0.4) (layers "F.Cu" "B.Cu") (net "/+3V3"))
 (via (at 57.5 23.75) (size 0.8) (drill 0.4) (layers "F.Cu" "B.Cu") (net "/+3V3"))
 (via (at 59.25 22) (size 0.8) (drill 0.4) (layers "F.Cu" "B.Cu") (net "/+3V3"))
 (via (at 73.25 22) (size 0.8) (drill 0.4) (layers "F.Cu" "B.Cu") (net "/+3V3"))
 (via (at 75 23.75) (size 0.8) (drill 0.4) (layers "F.Cu" "B.Cu") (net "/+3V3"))
 (via (at 37.5 23.75) (size 0.8) (drill 0.4) (layers "F.Cu" "B.Cu") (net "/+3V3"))
 (via (at 47.25 23) (size 0.8) (drill 0.4) (layers "F.Cu" "B.Cu") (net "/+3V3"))
 (via (at 135 23.75) (size 0.8) (drill 0.4) (layers "F.Cu" "B.Cu") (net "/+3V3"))
 (via (at 132.25 23) (size 0.8) (drill 0.4) (layers "F.Cu" "B.Cu") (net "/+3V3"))
 (via (at 101.25 24) (size 0.8) (drill 0.4) (layers "F.Cu" "B.Cu") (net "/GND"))
 (via (at 118.5 16.25) (size 0.8) (drill 0.4) (layers "F.Cu" "B.Cu") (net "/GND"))
 (via (at 91.25 14.5) (size 0.8) (drill 0.4) (layers "F.Cu" "B.Cu") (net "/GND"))
 (via (at 138.5 16.25) (size 0.8) (drill 0.4) (layers "F.Cu" "B.Cu") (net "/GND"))
 (via (at 38.75 14.5) (size 0.8) (drill 0.4) (layers "F.Cu" "B.Cu") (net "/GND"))
 (via (at 18.25 16.5) (size 0.8) (drill 0.4) (layers "F.Cu" "B.Cu") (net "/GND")))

